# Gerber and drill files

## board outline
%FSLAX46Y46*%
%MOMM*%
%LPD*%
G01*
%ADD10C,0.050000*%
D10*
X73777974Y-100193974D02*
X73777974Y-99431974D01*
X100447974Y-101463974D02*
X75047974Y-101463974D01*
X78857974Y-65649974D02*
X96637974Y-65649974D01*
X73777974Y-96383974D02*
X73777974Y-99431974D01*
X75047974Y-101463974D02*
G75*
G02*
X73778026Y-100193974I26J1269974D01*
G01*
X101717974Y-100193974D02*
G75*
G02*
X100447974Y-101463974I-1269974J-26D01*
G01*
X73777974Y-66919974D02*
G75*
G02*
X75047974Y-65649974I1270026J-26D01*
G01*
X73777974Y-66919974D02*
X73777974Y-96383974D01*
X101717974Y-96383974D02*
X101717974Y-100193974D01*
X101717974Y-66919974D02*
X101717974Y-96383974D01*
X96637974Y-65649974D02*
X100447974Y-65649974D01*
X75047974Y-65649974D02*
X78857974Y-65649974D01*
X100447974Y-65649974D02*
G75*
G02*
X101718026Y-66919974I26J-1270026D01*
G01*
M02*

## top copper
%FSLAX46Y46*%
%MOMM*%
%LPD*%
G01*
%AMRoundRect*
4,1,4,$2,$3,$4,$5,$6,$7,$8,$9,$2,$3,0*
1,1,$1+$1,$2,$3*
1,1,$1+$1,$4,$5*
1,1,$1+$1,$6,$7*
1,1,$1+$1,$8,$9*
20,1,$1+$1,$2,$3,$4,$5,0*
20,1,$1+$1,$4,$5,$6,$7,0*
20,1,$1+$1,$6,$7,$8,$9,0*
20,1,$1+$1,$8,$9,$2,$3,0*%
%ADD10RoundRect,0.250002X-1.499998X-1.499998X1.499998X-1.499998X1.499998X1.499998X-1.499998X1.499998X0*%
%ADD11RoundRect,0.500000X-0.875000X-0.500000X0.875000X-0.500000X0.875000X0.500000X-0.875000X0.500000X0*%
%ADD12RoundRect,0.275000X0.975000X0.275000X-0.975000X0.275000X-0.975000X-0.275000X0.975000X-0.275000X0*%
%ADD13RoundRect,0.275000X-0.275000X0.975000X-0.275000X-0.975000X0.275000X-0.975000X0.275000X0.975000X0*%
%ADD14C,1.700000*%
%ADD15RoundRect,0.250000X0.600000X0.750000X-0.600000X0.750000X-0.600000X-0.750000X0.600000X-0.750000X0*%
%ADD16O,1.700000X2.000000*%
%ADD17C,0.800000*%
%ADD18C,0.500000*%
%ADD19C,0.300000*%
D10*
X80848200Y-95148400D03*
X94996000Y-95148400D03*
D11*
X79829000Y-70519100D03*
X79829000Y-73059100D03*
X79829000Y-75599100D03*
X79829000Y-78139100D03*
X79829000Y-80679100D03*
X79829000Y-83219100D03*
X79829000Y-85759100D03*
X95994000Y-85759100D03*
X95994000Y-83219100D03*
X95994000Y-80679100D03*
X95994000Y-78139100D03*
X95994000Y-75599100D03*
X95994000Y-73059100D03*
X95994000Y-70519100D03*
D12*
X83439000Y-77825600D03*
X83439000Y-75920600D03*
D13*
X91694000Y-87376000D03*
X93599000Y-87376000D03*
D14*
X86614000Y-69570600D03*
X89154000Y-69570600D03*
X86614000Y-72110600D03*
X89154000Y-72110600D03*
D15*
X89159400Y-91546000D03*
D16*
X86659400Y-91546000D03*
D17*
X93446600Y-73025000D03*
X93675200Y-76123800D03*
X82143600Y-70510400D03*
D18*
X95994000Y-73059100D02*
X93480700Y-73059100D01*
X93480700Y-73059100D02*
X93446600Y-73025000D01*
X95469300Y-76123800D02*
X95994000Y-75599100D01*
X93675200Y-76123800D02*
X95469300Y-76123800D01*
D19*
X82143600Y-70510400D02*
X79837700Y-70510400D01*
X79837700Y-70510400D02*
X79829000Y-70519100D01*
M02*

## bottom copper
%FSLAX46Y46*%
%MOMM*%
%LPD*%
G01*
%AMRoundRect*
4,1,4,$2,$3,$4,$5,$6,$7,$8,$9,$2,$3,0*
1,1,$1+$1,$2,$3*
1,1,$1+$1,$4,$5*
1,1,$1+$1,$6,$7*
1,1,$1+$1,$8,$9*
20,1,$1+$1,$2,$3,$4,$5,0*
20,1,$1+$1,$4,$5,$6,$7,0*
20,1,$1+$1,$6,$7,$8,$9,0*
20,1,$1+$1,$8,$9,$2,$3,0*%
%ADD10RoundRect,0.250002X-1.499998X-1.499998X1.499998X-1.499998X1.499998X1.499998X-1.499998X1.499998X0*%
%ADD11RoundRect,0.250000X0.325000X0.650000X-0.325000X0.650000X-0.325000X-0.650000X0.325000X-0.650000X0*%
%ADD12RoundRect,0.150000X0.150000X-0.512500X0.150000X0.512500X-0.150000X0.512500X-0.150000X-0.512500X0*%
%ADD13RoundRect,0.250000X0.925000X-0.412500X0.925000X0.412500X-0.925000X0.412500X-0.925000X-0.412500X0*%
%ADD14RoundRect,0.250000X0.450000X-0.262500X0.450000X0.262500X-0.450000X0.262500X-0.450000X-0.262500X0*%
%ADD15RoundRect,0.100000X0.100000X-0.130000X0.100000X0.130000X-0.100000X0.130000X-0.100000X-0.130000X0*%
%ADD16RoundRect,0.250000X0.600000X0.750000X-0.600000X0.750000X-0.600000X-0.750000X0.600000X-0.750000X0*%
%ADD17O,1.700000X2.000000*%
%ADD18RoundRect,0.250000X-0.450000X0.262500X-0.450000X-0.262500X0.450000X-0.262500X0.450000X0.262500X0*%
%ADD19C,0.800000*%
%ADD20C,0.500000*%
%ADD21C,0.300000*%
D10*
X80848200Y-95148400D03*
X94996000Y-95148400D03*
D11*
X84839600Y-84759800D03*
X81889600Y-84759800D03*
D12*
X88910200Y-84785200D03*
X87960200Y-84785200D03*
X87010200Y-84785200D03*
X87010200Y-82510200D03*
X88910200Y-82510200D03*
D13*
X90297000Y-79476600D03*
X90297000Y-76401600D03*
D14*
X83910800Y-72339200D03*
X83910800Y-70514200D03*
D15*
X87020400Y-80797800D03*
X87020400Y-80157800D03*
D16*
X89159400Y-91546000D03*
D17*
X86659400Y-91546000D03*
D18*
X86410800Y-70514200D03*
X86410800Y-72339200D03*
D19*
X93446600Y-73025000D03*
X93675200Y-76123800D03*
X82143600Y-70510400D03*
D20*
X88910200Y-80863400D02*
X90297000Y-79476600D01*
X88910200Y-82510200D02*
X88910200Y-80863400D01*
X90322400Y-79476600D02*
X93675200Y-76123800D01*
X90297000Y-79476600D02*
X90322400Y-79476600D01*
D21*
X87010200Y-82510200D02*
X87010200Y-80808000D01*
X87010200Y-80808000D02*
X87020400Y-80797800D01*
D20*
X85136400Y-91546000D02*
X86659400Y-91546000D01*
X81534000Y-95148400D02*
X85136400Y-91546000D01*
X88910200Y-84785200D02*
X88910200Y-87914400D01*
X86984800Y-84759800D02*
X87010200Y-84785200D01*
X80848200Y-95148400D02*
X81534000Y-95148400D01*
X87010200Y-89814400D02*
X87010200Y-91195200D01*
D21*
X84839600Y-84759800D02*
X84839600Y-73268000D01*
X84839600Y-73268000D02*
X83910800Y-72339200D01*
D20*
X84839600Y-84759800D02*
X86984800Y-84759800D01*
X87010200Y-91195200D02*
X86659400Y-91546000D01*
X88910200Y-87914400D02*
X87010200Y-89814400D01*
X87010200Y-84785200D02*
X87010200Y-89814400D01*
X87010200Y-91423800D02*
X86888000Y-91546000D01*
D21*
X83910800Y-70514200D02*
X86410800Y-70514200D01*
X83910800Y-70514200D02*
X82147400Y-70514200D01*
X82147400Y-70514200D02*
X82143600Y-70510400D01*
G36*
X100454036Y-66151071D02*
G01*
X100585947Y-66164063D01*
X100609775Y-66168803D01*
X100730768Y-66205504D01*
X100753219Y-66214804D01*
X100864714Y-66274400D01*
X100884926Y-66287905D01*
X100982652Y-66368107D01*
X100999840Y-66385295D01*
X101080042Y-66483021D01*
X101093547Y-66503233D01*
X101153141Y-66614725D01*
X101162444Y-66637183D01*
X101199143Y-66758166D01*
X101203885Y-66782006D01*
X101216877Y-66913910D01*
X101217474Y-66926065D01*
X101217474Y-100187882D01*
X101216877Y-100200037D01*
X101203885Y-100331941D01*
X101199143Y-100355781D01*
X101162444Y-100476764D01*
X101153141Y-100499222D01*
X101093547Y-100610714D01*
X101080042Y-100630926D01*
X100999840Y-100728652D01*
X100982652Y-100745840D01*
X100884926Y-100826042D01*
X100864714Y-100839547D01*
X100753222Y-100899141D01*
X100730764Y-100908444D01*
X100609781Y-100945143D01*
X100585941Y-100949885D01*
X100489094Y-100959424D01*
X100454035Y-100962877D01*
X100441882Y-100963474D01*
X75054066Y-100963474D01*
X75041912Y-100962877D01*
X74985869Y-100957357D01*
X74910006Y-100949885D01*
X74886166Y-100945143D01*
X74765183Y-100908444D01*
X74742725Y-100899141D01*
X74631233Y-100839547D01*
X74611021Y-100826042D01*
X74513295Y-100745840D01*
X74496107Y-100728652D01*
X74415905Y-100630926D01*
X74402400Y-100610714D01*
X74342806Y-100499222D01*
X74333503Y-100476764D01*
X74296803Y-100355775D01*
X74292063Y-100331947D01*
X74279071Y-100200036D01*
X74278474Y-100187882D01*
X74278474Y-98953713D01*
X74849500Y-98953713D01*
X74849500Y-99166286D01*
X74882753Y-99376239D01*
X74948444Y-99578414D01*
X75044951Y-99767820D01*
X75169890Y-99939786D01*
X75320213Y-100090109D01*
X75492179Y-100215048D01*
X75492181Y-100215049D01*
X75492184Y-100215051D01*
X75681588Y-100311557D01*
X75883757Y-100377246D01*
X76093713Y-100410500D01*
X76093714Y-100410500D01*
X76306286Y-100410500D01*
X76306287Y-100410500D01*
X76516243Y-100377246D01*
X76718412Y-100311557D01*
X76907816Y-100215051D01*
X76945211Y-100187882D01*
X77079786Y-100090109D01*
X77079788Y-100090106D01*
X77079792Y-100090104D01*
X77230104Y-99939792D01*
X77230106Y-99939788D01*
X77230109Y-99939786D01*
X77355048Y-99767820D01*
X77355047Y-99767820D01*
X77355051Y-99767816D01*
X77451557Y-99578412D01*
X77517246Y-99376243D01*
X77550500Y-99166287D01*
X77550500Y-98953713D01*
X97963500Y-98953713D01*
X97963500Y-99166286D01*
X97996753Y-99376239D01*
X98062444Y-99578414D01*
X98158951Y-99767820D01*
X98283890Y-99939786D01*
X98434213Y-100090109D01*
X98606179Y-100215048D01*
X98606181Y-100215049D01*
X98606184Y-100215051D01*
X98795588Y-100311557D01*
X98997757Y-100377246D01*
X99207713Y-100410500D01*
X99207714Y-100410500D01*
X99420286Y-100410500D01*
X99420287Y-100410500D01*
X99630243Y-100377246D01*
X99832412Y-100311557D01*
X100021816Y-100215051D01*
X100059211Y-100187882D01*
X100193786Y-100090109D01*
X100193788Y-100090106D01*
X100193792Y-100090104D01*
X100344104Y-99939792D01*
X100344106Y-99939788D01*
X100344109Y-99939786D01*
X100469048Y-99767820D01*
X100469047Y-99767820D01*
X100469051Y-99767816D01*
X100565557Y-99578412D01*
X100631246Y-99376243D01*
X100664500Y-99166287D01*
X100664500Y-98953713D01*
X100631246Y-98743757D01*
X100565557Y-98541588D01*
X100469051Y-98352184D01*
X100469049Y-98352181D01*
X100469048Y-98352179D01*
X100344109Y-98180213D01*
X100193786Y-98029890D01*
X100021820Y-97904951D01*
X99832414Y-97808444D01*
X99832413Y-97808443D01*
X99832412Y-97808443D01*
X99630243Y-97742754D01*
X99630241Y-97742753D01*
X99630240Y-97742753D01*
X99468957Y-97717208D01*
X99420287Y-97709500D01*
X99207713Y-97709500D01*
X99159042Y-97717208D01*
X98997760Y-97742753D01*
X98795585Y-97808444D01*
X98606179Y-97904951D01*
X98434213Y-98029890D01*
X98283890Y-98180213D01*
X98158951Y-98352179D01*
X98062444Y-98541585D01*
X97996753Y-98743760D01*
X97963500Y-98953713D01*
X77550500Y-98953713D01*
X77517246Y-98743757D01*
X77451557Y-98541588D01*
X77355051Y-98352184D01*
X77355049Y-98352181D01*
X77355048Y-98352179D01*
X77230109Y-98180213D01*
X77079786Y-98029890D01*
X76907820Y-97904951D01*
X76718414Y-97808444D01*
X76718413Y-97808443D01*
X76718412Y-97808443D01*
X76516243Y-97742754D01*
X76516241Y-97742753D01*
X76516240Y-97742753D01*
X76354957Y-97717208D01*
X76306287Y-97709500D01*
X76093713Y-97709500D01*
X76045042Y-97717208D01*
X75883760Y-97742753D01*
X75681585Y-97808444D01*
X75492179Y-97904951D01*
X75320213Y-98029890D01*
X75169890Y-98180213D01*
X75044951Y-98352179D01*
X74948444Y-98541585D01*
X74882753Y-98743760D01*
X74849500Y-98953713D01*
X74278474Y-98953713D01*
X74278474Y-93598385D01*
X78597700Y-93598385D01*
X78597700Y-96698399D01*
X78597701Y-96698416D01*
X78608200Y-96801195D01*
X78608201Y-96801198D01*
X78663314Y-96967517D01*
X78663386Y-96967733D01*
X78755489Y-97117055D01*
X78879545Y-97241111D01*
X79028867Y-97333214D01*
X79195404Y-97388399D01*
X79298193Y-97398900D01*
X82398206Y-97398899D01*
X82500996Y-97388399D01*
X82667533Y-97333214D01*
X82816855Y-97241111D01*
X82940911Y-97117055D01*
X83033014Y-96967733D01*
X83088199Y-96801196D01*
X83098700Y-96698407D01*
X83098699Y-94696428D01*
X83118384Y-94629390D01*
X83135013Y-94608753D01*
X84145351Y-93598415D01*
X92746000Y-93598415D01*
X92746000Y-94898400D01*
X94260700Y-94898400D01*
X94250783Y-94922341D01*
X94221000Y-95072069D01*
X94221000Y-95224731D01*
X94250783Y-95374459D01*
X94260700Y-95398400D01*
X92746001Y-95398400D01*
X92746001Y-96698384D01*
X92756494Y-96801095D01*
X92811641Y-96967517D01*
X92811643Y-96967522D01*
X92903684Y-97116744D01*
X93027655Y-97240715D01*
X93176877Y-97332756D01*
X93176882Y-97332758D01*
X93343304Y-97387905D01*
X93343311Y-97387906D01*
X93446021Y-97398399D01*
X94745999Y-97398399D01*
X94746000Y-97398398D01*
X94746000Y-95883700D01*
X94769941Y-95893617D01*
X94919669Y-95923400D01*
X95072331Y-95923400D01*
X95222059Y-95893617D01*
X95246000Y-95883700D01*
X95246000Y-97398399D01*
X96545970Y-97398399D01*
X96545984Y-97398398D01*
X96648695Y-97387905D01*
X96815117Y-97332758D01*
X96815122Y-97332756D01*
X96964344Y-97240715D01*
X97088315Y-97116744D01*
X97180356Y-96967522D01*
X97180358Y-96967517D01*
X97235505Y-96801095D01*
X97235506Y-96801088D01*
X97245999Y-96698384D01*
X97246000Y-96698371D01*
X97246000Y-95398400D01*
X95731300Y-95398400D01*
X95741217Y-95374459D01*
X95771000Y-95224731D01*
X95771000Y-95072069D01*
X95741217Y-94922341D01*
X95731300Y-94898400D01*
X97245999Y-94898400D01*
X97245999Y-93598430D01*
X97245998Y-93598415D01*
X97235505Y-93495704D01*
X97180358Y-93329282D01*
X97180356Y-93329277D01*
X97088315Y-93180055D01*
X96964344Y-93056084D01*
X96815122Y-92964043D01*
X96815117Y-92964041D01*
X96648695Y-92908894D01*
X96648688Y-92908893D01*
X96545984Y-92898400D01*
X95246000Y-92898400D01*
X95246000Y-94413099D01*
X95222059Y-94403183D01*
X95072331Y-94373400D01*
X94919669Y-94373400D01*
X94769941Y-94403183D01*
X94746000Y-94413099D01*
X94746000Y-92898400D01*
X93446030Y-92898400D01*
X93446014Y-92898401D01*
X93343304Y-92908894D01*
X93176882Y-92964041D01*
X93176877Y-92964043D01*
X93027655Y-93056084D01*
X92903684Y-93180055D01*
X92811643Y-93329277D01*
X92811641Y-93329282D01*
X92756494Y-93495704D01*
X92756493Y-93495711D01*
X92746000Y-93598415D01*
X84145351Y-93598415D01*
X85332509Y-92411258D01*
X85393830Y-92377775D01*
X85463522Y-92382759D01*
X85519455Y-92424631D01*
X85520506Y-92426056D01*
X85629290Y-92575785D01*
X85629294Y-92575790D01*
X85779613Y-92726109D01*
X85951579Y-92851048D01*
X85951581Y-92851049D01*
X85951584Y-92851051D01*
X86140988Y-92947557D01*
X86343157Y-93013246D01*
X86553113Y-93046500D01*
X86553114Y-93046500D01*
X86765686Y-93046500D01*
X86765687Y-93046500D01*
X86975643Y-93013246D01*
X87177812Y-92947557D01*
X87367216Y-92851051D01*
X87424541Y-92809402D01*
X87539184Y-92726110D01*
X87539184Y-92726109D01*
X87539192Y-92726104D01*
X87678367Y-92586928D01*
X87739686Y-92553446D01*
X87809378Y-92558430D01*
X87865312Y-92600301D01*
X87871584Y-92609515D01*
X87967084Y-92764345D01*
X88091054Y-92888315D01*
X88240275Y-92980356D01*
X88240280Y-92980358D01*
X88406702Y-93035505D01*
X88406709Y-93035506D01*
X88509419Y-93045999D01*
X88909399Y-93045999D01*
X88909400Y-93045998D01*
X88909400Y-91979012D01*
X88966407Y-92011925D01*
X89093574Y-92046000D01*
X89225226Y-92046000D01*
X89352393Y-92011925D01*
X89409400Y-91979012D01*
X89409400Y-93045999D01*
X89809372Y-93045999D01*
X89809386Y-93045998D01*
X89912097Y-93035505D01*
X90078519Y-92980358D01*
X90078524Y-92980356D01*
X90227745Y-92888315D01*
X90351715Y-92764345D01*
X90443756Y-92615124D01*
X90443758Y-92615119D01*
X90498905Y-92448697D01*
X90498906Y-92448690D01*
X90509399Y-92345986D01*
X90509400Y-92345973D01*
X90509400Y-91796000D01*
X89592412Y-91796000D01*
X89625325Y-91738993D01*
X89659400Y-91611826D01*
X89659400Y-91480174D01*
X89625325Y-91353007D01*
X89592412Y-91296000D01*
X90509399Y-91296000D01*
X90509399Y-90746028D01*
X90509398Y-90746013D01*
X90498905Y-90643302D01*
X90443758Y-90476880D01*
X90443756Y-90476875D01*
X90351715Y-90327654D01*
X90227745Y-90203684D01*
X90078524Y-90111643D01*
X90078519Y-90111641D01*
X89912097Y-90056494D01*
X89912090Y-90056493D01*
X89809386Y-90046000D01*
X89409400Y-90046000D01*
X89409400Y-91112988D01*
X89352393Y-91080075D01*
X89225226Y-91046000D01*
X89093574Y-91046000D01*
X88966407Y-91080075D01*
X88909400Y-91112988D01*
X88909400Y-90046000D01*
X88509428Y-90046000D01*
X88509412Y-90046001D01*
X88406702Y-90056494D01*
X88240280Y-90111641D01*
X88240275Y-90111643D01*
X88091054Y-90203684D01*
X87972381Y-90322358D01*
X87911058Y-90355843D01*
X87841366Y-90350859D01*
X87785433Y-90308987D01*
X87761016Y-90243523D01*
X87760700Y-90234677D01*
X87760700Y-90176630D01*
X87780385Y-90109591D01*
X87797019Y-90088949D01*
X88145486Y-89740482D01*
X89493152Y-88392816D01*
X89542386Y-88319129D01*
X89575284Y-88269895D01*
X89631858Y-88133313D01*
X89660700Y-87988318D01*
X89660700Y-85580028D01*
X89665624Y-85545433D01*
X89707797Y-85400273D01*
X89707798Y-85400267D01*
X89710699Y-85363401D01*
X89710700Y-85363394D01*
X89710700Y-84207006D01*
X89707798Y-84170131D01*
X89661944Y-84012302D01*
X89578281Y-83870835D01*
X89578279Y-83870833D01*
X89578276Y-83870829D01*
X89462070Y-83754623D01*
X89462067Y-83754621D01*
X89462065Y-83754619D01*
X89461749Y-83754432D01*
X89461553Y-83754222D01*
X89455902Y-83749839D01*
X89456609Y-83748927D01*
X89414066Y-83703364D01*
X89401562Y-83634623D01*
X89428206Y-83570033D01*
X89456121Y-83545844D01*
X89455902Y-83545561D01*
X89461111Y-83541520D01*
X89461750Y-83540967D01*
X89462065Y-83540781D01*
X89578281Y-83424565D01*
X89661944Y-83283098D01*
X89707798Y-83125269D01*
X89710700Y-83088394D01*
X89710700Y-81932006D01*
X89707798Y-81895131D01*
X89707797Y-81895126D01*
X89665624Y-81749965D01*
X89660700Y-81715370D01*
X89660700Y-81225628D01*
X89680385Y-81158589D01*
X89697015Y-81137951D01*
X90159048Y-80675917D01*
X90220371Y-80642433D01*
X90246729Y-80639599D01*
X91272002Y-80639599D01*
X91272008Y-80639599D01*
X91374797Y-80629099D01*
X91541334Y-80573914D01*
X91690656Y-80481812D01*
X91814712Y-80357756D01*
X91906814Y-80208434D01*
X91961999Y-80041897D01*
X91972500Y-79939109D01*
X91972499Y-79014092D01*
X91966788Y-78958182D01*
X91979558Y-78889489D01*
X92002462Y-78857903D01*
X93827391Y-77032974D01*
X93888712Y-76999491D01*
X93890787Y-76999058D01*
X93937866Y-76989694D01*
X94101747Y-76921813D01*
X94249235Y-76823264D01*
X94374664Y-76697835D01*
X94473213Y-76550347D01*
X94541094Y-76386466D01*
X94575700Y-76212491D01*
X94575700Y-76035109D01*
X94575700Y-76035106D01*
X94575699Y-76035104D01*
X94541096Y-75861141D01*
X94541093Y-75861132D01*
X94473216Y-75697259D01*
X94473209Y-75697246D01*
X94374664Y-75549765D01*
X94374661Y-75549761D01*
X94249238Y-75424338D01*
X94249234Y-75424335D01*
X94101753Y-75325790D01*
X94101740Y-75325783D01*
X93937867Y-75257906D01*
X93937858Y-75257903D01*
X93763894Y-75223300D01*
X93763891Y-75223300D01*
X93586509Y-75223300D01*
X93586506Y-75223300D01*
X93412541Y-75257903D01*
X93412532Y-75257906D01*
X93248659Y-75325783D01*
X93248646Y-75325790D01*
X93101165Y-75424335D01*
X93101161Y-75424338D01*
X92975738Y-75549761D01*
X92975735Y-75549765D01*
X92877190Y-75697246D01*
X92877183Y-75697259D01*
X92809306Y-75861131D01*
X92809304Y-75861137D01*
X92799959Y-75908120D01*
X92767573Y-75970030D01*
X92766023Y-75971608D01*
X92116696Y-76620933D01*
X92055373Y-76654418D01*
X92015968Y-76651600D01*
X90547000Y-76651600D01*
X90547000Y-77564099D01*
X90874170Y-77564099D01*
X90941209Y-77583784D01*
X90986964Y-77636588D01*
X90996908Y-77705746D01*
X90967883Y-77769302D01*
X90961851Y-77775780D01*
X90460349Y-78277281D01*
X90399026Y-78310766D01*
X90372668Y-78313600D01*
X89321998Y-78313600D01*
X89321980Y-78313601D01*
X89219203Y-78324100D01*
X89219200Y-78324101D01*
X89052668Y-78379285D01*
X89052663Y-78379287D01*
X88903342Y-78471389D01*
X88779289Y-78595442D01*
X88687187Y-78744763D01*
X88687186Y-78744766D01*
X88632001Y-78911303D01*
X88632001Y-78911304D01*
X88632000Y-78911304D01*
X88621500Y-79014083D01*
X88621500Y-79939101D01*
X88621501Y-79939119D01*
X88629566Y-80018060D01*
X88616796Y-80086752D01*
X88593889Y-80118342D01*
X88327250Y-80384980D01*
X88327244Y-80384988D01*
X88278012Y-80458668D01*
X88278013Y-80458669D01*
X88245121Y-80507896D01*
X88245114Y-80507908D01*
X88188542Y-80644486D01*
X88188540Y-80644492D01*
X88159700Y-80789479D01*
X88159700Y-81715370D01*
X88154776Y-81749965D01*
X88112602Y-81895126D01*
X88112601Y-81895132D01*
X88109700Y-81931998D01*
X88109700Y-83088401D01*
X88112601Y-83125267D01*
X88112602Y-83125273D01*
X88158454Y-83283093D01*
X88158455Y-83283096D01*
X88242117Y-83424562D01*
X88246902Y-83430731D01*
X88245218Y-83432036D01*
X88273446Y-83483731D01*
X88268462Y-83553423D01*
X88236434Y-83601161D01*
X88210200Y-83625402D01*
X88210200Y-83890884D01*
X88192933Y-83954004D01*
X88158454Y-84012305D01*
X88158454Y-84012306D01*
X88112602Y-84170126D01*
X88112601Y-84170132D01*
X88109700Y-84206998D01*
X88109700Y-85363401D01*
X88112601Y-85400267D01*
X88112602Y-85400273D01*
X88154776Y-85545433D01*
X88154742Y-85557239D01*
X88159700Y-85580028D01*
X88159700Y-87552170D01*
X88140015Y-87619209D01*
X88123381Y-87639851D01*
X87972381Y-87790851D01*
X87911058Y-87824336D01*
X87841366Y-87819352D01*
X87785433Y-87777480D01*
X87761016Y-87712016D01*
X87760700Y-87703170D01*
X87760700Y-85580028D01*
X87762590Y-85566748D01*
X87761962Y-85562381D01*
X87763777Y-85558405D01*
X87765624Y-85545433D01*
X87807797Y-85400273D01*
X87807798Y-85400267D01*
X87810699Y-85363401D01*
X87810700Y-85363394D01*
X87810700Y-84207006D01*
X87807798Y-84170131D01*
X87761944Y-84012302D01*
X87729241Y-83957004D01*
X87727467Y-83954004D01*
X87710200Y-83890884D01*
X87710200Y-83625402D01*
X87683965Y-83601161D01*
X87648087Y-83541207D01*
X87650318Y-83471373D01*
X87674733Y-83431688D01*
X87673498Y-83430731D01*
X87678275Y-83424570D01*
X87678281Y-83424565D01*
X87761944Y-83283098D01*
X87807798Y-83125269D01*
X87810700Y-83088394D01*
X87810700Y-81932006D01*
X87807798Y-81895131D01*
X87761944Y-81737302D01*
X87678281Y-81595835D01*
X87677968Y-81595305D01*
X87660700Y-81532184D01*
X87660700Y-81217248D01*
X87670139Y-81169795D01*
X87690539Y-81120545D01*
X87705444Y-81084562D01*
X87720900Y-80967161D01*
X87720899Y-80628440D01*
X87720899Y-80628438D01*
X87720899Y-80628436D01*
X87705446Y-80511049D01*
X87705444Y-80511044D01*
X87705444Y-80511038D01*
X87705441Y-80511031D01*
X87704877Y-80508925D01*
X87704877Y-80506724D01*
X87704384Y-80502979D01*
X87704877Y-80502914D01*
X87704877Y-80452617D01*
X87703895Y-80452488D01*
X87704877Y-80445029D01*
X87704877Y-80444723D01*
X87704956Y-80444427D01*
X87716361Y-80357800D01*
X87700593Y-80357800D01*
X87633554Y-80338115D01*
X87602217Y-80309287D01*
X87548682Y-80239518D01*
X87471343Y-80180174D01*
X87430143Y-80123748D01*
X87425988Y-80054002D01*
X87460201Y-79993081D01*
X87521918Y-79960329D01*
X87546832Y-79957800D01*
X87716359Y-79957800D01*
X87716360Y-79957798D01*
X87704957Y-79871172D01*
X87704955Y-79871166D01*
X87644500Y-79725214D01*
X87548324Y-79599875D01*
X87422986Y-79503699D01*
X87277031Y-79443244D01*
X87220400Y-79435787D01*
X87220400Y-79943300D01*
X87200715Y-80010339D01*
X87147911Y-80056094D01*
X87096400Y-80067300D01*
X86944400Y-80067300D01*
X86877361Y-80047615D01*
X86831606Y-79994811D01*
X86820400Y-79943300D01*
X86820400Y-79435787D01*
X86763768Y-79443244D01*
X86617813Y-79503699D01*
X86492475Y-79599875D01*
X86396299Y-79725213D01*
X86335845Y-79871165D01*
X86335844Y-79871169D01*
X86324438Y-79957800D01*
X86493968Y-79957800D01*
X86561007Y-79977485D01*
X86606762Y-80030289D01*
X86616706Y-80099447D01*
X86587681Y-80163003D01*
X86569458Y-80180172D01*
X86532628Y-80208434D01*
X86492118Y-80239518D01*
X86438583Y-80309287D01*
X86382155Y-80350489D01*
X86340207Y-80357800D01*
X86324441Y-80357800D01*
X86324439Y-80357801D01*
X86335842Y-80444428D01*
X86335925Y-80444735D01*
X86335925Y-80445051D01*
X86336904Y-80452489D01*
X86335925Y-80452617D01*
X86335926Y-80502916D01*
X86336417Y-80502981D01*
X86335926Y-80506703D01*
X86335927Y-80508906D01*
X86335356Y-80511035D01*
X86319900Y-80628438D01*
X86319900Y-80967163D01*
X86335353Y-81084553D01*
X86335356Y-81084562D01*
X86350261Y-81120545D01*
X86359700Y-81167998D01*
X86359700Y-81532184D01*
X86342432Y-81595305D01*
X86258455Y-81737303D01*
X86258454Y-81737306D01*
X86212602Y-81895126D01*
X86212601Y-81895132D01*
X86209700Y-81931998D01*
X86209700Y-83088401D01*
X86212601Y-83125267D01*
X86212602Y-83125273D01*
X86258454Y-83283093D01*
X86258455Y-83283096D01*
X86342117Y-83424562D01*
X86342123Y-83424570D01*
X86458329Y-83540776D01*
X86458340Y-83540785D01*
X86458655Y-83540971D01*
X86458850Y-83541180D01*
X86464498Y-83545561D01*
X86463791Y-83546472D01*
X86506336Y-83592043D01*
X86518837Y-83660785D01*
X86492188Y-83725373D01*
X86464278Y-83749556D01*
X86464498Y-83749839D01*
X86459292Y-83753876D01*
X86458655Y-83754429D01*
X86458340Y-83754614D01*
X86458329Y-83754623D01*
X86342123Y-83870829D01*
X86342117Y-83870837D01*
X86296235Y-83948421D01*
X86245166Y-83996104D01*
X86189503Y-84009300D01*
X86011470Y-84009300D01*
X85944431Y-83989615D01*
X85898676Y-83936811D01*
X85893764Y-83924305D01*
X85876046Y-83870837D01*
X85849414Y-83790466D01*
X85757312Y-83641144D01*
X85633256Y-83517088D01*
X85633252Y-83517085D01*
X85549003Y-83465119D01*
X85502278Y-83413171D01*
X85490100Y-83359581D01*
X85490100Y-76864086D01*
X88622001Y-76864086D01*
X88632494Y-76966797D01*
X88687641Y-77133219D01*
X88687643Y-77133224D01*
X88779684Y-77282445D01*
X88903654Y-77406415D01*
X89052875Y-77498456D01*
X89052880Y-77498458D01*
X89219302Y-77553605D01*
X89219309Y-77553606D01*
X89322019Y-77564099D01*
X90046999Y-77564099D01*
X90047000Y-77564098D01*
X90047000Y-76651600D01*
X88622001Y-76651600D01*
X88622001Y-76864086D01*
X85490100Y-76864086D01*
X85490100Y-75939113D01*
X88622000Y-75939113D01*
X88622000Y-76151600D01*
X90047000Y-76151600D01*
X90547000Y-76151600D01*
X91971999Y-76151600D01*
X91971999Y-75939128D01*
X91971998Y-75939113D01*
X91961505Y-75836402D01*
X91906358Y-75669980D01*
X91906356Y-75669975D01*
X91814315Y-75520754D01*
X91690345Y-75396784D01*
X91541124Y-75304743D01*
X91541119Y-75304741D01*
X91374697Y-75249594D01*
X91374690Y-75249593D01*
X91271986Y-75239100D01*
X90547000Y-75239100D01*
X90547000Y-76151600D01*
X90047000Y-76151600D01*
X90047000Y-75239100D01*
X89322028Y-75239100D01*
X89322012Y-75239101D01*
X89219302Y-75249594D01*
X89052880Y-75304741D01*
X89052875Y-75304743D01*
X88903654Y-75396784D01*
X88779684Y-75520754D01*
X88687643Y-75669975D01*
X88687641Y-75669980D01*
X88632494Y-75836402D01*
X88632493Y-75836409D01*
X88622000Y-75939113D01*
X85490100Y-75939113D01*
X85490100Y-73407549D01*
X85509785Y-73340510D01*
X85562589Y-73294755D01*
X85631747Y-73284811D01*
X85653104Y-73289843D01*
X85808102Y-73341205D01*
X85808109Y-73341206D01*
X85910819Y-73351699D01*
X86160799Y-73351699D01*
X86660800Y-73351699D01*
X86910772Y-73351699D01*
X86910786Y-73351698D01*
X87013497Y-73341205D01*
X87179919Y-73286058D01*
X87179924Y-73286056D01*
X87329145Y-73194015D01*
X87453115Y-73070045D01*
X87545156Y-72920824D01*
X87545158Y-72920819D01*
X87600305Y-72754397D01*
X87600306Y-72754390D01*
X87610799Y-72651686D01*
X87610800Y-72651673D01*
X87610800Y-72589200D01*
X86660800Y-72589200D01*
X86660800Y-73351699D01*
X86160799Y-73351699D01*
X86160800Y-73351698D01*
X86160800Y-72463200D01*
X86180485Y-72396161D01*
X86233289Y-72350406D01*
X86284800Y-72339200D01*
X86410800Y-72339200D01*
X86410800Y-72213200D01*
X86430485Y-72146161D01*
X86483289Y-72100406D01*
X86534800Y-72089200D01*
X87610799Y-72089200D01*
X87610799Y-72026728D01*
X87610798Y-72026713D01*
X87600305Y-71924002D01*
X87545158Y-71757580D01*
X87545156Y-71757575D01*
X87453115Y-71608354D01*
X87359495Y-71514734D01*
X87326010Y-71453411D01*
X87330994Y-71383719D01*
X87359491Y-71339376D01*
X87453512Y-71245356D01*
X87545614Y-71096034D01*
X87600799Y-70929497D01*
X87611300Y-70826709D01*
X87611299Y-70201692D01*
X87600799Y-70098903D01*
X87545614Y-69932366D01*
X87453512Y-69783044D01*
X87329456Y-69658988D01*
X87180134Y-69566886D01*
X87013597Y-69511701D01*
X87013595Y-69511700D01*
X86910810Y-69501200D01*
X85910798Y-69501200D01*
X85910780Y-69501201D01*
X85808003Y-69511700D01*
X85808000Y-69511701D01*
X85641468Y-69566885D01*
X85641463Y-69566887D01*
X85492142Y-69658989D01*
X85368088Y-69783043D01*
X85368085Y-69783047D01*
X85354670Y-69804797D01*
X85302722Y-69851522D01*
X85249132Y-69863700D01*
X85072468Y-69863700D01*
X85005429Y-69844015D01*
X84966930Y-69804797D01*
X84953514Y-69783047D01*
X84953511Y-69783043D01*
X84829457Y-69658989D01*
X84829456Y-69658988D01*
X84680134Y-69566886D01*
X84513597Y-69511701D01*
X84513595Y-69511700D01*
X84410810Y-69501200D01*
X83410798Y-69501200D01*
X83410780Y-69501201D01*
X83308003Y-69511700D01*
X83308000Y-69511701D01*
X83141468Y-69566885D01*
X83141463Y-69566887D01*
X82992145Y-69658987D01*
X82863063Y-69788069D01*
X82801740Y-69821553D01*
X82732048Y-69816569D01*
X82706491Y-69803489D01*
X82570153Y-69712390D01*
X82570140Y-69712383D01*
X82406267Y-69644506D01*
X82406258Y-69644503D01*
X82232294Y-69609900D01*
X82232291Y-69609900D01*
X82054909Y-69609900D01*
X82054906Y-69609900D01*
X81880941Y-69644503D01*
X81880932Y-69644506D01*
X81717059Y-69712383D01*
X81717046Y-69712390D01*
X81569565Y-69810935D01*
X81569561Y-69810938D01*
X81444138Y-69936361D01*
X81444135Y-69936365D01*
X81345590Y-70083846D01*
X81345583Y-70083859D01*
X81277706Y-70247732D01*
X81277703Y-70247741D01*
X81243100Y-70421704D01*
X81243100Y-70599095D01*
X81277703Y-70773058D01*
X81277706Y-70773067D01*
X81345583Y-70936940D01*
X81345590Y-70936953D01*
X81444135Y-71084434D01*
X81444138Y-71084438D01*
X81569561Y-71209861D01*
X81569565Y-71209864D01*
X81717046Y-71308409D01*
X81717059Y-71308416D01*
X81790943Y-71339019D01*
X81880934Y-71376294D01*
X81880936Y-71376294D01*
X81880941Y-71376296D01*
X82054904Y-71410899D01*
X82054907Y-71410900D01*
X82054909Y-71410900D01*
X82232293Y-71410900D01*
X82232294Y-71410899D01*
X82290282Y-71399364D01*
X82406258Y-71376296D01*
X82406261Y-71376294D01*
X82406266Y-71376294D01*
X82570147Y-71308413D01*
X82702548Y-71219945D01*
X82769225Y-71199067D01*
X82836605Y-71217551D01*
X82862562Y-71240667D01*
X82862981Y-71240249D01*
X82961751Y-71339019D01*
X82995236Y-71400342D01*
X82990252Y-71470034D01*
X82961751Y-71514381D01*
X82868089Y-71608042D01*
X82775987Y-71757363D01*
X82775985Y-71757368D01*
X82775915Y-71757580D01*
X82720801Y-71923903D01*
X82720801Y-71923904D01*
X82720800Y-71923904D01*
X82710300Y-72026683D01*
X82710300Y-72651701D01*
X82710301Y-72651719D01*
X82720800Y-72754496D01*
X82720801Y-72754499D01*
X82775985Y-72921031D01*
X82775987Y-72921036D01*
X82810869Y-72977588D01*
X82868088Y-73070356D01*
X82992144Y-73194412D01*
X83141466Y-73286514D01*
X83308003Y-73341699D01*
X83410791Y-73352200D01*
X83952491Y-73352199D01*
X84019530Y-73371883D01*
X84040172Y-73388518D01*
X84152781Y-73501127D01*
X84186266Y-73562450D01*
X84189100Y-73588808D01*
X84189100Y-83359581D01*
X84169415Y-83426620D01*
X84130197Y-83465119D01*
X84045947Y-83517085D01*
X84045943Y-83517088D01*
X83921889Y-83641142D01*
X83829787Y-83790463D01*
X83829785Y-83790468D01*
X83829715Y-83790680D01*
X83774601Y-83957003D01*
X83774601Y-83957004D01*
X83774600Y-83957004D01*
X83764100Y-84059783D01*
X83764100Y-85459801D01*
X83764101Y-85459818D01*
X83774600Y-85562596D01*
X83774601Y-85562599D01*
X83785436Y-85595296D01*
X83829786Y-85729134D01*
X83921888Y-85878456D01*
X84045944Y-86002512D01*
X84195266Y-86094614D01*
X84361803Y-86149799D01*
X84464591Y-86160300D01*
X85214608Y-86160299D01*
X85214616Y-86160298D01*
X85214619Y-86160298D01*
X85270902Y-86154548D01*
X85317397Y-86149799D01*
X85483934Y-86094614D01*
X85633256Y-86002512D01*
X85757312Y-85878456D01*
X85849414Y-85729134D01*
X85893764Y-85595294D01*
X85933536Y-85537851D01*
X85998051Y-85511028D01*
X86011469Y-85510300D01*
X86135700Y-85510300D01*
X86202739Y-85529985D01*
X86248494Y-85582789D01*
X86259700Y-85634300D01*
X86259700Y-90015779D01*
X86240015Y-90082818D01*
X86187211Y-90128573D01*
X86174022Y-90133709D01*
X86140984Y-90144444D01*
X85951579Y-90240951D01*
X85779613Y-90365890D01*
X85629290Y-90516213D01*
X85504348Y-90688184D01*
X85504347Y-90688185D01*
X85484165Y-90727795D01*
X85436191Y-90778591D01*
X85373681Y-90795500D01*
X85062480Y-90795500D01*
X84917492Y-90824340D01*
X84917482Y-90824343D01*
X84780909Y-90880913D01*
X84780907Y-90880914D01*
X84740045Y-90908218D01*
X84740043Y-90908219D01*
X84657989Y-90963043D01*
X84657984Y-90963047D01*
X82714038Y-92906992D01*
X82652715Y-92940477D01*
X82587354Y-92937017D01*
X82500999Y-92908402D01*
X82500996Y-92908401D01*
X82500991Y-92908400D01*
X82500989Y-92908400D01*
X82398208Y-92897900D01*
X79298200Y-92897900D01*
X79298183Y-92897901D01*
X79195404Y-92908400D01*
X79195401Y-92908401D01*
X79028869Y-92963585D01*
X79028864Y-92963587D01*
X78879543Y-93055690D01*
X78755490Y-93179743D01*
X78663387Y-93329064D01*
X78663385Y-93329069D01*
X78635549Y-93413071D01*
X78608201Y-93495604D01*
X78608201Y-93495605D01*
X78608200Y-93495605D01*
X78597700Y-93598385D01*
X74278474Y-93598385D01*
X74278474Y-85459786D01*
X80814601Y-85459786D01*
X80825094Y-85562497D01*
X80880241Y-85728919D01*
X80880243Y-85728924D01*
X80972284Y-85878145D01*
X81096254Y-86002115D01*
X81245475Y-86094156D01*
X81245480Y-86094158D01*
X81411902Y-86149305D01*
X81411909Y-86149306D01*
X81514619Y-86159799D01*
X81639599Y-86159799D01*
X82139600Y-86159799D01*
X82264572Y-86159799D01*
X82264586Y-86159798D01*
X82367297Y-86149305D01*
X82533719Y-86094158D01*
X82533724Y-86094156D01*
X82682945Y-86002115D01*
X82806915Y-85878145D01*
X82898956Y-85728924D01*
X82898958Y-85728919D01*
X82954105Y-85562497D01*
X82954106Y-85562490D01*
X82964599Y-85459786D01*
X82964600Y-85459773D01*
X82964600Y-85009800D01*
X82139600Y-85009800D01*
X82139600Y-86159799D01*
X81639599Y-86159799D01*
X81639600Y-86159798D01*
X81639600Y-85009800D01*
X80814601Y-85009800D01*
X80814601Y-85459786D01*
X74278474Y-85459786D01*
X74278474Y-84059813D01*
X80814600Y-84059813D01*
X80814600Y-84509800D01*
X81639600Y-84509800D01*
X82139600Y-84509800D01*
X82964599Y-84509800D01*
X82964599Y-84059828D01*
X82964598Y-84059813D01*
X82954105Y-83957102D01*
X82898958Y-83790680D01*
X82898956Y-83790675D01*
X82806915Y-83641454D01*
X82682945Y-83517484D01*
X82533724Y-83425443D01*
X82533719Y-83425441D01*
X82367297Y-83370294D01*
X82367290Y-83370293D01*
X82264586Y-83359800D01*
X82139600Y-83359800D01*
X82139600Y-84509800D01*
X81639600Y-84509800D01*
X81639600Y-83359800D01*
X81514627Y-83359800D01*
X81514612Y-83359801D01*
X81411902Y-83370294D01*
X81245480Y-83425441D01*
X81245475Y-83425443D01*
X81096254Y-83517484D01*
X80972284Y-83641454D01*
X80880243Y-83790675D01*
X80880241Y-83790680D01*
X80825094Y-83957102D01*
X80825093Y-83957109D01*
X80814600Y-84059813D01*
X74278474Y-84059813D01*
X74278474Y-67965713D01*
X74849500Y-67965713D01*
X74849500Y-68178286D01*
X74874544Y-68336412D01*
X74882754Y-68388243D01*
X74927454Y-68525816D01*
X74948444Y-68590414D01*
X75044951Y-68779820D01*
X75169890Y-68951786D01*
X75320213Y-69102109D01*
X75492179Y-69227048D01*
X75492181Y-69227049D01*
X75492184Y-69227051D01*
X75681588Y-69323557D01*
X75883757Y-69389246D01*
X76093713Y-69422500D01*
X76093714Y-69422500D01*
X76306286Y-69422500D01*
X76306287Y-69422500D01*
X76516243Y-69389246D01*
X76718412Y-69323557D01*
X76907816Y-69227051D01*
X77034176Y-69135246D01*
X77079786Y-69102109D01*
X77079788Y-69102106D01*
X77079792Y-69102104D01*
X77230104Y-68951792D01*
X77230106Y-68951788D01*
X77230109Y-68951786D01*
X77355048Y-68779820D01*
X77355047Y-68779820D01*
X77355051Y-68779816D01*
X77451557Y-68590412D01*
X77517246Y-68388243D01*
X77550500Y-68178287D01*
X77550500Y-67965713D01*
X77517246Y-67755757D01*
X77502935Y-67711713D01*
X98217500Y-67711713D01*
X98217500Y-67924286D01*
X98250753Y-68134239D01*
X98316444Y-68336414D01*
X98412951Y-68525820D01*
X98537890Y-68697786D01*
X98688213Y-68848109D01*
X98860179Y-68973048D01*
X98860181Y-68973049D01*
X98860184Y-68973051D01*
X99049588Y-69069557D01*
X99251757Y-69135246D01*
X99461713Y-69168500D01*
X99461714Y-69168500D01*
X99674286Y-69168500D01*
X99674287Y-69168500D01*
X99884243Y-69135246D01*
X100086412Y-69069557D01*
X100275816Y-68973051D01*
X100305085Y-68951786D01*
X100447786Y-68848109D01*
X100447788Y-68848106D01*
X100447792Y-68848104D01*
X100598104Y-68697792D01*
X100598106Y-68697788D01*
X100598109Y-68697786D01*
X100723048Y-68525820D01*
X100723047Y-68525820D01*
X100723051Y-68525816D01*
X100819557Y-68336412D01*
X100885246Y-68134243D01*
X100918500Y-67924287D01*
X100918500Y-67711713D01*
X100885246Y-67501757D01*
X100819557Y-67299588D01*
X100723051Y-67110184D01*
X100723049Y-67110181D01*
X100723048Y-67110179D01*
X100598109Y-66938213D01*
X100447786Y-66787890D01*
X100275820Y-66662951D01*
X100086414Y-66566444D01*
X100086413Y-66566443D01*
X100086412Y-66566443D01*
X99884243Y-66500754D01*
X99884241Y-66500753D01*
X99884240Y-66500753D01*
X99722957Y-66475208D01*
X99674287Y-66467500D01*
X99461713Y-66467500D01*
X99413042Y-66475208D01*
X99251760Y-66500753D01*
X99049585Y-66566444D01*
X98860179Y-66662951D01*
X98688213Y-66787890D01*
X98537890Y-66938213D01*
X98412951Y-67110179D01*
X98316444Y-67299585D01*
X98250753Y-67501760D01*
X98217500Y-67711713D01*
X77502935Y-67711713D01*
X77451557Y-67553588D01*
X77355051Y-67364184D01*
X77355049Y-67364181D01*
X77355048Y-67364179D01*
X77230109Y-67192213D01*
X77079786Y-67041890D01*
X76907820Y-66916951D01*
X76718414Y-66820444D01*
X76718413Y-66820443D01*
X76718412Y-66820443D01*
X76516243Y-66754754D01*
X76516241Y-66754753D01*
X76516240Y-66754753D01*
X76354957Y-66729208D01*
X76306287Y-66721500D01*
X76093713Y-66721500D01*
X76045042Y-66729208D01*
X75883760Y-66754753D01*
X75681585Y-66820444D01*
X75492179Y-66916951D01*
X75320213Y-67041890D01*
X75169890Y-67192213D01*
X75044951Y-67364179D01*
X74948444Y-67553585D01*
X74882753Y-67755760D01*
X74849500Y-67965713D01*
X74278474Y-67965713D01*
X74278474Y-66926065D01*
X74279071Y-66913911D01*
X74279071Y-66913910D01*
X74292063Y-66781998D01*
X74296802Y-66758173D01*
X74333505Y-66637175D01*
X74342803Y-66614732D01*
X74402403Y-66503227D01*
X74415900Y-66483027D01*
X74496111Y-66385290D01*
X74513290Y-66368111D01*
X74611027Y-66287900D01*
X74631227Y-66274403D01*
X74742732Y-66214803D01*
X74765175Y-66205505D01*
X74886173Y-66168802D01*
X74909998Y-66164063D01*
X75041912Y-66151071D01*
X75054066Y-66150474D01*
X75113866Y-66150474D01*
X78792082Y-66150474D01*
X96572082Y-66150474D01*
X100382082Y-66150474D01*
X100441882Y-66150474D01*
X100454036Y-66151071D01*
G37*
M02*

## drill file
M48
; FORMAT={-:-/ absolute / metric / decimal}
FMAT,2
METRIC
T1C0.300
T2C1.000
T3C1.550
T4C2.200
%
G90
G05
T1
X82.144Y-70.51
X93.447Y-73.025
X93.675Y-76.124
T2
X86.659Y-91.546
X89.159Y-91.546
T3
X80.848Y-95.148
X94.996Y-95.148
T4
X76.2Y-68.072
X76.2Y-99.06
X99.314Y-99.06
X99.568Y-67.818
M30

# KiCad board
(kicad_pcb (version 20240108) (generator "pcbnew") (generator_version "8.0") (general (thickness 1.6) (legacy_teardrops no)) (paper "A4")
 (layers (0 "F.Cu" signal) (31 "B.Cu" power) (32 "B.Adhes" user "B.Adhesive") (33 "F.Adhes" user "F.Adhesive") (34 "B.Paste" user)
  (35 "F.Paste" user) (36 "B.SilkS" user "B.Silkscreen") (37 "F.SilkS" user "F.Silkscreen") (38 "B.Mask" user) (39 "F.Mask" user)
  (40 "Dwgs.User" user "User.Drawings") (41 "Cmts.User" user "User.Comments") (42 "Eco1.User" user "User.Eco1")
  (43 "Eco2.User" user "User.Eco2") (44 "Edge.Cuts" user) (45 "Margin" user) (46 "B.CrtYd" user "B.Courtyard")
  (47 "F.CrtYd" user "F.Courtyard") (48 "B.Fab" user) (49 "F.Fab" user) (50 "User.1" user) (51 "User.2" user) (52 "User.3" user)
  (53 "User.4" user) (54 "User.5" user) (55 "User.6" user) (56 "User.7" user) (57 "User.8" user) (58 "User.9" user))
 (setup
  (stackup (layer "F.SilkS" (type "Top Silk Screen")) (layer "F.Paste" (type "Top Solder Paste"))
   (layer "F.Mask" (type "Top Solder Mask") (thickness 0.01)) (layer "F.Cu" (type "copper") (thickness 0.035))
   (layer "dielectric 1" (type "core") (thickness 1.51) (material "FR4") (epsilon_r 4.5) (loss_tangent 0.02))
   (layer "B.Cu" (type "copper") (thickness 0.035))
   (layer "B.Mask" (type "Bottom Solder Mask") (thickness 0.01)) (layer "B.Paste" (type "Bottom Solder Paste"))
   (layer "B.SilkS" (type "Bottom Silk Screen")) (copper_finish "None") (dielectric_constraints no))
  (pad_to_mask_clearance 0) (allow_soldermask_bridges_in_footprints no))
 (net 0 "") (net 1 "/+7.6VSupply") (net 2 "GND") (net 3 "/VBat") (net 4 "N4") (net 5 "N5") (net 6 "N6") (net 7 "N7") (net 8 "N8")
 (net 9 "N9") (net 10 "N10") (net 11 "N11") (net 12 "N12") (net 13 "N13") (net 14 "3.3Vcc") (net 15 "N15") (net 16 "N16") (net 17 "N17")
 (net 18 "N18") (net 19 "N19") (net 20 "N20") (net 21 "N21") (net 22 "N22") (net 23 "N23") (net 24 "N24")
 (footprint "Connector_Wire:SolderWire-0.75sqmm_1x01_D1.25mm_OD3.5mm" (layer "F.Cu") (at 80.8482 95.1484)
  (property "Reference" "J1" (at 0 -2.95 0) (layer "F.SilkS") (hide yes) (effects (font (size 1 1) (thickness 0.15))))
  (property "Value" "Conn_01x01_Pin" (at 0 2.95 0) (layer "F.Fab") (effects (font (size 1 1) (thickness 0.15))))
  (pad "1" thru_hole roundrect (at 0 0) (size 3.5 3.5) (drill 1.55) (layers "*.Cu" "*.Mask") (remove_unused_layers no)
   (roundrect_rratio 0.071429) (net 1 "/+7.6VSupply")))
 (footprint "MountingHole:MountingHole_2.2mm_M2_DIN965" (layer "F.Cu") (at 99.568 67.818)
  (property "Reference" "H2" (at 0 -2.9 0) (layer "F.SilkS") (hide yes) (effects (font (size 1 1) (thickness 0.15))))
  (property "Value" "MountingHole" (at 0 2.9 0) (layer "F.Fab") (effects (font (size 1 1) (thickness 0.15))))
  (pad "" np_thru_hole circle (at 0 0) (size 2.2 2.2) (drill 2.2) (layers "*.Cu" "*.Mask")))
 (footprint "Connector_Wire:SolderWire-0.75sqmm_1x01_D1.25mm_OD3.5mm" (layer "F.Cu") (at 94.996 95.1484)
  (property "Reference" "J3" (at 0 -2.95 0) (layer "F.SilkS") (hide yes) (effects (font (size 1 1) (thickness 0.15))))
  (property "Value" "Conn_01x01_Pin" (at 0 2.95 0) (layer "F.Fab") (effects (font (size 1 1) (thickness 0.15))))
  (pad "1" thru_hole roundrect (at 0 0) (size 3.5 3.5) (drill 1.55) (layers "*.Cu" "*.Mask") (remove_unused_layers no)
   (roundrect_rratio 0.071429) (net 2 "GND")))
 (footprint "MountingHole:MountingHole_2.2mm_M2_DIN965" (layer "F.Cu") (at 76.2 99.06)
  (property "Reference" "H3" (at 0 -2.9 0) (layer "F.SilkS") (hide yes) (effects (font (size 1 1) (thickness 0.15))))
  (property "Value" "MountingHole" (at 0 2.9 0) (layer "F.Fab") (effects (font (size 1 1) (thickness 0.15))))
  (pad "" np_thru_hole circle (at 0 0) (size 2.2 2.2) (drill 2.2) (layers "*.Cu" "*.Mask")))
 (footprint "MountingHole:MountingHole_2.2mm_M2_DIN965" (layer "F.Cu") (at 99.314 99.06)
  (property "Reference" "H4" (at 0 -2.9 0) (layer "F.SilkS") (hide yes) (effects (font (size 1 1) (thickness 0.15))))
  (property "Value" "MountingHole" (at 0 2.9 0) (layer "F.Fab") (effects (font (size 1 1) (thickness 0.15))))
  (pad "" np_thru_hole circle (at 0 0) (size 2.2 2.2) (drill 2.2) (layers "*.Cu" "*.Mask")))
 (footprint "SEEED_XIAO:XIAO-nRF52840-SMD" (layer "F.Cu") (at 78.994 88.6391)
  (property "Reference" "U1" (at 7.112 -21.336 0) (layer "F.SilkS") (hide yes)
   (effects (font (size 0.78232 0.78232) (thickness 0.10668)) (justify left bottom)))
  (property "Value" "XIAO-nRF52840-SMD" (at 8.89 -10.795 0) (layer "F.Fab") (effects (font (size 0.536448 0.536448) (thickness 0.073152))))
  (pad "1" smd roundrect (at 0.835 -18.12) (size 2.75 2) (layers "F.Cu" "F.Paste" "F.Mask") (roundrect_rratio 0.25) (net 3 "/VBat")
   (solder_mask_margin 0.0508) (thermal_bridge_angle 45))
  (pad "2" smd roundrect (at 0.835 -15.58) (size 2.75 2) (layers "F.Cu" "F.Paste" "F.Mask") (roundrect_rratio 0.25) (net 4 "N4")
   (solder_mask_margin 0.0508) (thermal_bridge_angle 45))
  (pad "3" smd roundrect (at 0.835 -13.04) (size 2.75 2) (layers "F.Cu" "F.Paste" "F.Mask") (roundrect_rratio 0.25) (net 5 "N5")
   (solder_mask_margin 0.0508) (thermal_bridge_angle 45))
  (pad "4" smd roundrect (at 0.835 -10.5) (size 2.75 2) (layers "F.Cu" "F.Paste" "F.Mask") (roundrect_rratio 0.25) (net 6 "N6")
   (solder_mask_margin 0.0508) (thermal_bridge_angle 45))
  (pad "5" smd roundrect (at 0.835 -7.96) (size 2.75 2) (layers "F.Cu" "F.Paste" "F.Mask") (roundrect_rratio 0.25) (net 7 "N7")
   (solder_mask_margin 0.0508) (thermal_bridge_angle 45))
  (pad "6" smd roundrect (at 0.835 -5.42) (size 2.75 2) (layers "F.Cu" "F.Paste" "F.Mask") (roundrect_rratio 0.25) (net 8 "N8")
   (solder_mask_margin 0.0508) (thermal_bridge_angle 45))
  (pad "7" smd roundrect (at 0.835 -2.88) (size 2.75 2) (layers "F.Cu" "F.Paste" "F.Mask") (roundrect_rratio 0.25) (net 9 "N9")
   (solder_mask_margin 0.0508) (thermal_bridge_angle 45))
  (pad "8" smd roundrect (at 17 -2.88) (size 2.75 2) (layers "F.Cu" "F.Paste" "F.Mask") (roundrect_rratio 0.25) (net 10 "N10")
   (solder_mask_margin 0.0508) (thermal_bridge_angle 45))
  (pad "9" smd roundrect (at 17 -5.42) (size 2.75 2) (layers "F.Cu" "F.Paste" "F.Mask") (roundrect_rratio 0.25) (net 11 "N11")
   (solder_mask_margin 0.0508) (thermal_bridge_angle 45))
  (pad "10" smd roundrect (at 17 -7.96) (size 2.75 2) (layers "F.Cu" "F.Paste" "F.Mask") (roundrect_rratio 0.25) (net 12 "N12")
   (solder_mask_margin 0.0508) (thermal_bridge_angle 45))
  (pad "11" smd roundrect (at 17 -10.5) (size 2.75 2) (layers "F.Cu" "F.Paste" "F.Mask") (roundrect_rratio 0.25) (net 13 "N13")
   (solder_mask_margin 0.0508) (thermal_bridge_angle 45))
  (pad "12" smd roundrect (at 17 -13.04) (size 2.75 2) (layers "F.Cu" "F.Paste" "F.Mask") (roundrect_rratio 0.25) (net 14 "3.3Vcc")
   (solder_mask_margin 0.0508) (thermal_bridge_angle 45))
  (pad "13" smd roundrect (at 17 -15.58) (size 2.75 2) (layers "F.Cu" "F.Paste" "F.Mask") (roundrect_rratio 0.25) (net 2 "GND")
   (solder_mask_margin 0.0508) (thermal_bridge_angle 45))
  (pad "14" smd roundrect (at 17 -18.12) (size 2.75 2) (layers "F.Cu" "F.Paste" "F.Mask") (roundrect_rratio 0.25) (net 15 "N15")
   (solder_mask_margin 0.0508) (thermal_bridge_angle 45))
  (pad "15" smd roundrect (at 4.445 -10.8135 180) (size 2.5 1.1) (layers "F.Cu" "F.Paste" "F.Mask") (roundrect_rratio 0.25) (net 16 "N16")
   (solder_mask_margin 0.0508) (thermal_bridge_angle 45))
  (pad "16" smd roundrect (at 4.445 -12.7185 180) (size 2.5 1.1) (layers "F.Cu" "F.Paste" "F.Mask") (roundrect_rratio 0.25) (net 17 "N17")
   (solder_mask_margin 0.0508) (thermal_bridge_angle 45))
  (pad "17" smd roundrect (at 12.7 -1.2631 270) (size 2.5 1.1) (layers "F.Cu" "F.Paste" "F.Mask") (roundrect_rratio 0.25) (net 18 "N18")
   (solder_mask_margin 0.0508) (thermal_bridge_angle 45))
  (pad "18" smd roundrect (at 14.605 -1.2631 270) (size 2.5 1.1) (layers "F.Cu" "F.Paste" "F.Mask") (roundrect_rratio 0.25) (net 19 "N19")
   (solder_mask_margin 0.0508) (thermal_bridge_angle 45))
  (pad "19" smd circle (at 7.62 -19.0685) (size 1.7 1.7) (layers "F.Cu" "F.Paste" "F.Mask") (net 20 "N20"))
  (pad "20" smd circle (at 10.16 -19.0685) (size 1.7 1.7) (layers "F.Cu" "F.Paste" "F.Mask") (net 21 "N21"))
  (pad "21" smd circle (at 7.62 -16.5285) (size 1.7 1.7) (layers "F.Cu" "F.Paste" "F.Mask") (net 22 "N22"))
  (pad "22" smd circle (at 10.16 -16.5285) (size 1.7 1.7) (layers "F.Cu" "F.Paste" "F.Mask") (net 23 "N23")))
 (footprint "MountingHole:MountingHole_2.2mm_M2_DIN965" (layer "F.Cu") (at 76.2 68.072)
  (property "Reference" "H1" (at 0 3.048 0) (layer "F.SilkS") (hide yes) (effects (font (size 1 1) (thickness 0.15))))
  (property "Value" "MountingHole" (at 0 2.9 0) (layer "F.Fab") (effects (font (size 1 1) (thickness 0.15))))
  (pad "" np_thru_hole circle (at 0 0) (size 2.2 2.2) (drill 2.2) (layers "*.Cu" "*.Mask")))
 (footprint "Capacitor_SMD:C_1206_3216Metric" (layer "B.Cu") (at 83.3646 84.7598 180)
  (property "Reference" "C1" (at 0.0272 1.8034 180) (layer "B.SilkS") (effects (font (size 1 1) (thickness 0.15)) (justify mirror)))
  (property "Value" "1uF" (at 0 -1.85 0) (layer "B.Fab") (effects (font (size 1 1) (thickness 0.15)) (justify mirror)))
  (pad "1" smd roundrect (at -1.475 0 180) (size 1.15 1.8) (layers "B.Cu" "B.Paste" "B.Mask") (roundrect_rratio 0.217391)
   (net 1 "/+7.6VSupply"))
  (pad "2" smd roundrect (at 1.475 0 180) (size 1.15 1.8) (layers "B.Cu" "B.Paste" "B.Mask") (roundrect_rratio 0.217391) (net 2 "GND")))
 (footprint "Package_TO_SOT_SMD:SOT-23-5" (layer "B.Cu") (at 87.9602 83.6477 90)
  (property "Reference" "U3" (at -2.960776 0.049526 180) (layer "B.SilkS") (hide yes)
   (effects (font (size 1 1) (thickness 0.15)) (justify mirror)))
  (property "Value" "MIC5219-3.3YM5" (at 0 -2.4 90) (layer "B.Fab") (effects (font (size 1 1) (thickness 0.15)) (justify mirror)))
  (pad "1" smd roundrect (at -1.1375 0.95 90) (size 1.325 0.6) (layers "B.Cu" "B.Paste" "B.Mask") (roundrect_rratio 0.25)
   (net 1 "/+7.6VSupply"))
  (pad "2" smd roundrect (at -1.1375 0 90) (size 1.325 0.6) (layers "B.Cu" "B.Paste" "B.Mask") (roundrect_rratio 0.25) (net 2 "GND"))
  (pad "3" smd roundrect (at -1.1375 -0.95 90) (size 1.325 0.6) (layers "B.Cu" "B.Paste" "B.Mask") (roundrect_rratio 0.25)
   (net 1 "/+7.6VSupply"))
  (pad "4" smd roundrect (at 1.1375 -0.95 90) (size 1.325 0.6) (layers "B.Cu" "B.Paste" "B.Mask") (roundrect_rratio 0.25) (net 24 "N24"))
  (pad "5" smd roundrect (at 1.1375 0.95 90) (size 1.325 0.6) (layers "B.Cu" "B.Paste" "B.Mask") (roundrect_rratio 0.25) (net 14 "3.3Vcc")))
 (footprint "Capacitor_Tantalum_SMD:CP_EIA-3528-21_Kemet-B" (layer "B.Cu") (at 90.297 77.9391 90)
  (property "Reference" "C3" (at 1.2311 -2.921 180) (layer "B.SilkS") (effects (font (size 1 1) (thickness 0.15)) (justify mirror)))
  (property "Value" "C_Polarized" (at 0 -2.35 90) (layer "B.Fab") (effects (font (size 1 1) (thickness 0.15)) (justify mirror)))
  (pad "1" smd roundrect (at -1.5375 0 90) (size 1.325 2.35) (layers "B.Cu" "B.Paste" "B.Mask") (roundrect_rratio 0.188679)
   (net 14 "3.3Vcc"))
  (pad "2" smd roundrect (at 1.5375 0 90) (size 1.325 2.35) (layers "B.Cu" "B.Paste" "B.Mask") (roundrect_rratio 0.188679) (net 2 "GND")))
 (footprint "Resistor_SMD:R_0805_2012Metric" (layer "B.Cu") (at 83.9108 71.4267 90)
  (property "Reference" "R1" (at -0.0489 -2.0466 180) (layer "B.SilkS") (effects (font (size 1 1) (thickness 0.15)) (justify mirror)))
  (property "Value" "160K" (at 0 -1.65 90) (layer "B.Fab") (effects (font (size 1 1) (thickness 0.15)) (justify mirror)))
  (pad "1" smd roundrect (at -0.9125 0 90) (size 1.025 1.4) (layers "B.Cu" "B.Paste" "B.Mask") (roundrect_rratio 0.243902)
   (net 1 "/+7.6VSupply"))
  (pad "2" smd roundrect (at 0.9125 0 90) (size 1.025 1.4) (layers "B.Cu" "B.Paste" "B.Mask") (roundrect_rratio 0.243902) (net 3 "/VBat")))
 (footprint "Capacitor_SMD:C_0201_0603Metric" (layer "B.Cu") (at 87.0204 80.4778 90)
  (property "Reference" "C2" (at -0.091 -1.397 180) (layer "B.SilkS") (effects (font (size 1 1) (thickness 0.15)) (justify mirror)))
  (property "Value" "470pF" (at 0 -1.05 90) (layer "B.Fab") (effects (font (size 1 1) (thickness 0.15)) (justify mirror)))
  (pad "" smd roundrect (at -0.345 0 90) (size 0.318 0.36) (layers "B.Paste") (roundrect_rratio 0.25))
  (pad "" smd roundrect (at 0.345 0 90) (size 0.318 0.36) (layers "B.Paste") (roundrect_rratio 0.25))
  (pad "1" smd roundrect (at -0.32 0 90) (size 0.46 0.4) (layers "B.Cu" "B.Mask") (roundrect_rratio 0.25) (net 24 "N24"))
  (pad "2" smd roundrect (at 0.32 0 90) (size 0.46 0.4) (layers "B.Cu" "B.Mask") (roundrect_rratio 0.25) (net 2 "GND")))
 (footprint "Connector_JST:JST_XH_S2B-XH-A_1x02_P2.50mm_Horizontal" (layer "B.Cu") (at 89.1594 91.546 180)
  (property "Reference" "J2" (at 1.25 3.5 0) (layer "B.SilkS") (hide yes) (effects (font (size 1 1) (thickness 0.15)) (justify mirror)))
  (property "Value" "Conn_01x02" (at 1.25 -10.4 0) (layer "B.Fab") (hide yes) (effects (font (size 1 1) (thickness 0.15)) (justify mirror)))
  (pad "1" thru_hole roundrect (at 0 0 180) (size 1.7 2) (drill 1) (layers "*.Cu" "*.Mask") (remove_unused_layers no)
   (roundrect_rratio 0.147059) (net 2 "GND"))
  (pad "2" thru_hole oval (at 2.5 0 180) (size 1.7 2) (drill 1) (layers "*.Cu" "*.Mask") (remove_unused_layers no) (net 1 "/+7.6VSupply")))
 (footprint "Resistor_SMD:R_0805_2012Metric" (layer "B.Cu") (at 86.4108 71.4267 -90)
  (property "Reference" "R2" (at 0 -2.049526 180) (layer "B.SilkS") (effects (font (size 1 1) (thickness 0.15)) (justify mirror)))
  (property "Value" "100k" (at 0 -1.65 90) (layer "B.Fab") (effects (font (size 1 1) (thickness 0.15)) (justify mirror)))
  (pad "1" smd roundrect (at -0.9125 0 270) (size 1.025 1.4) (layers "B.Cu" "B.Paste" "B.Mask") (roundrect_rratio 0.243902) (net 3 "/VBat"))
  (pad "2" smd roundrect (at 0.9125 0 270) (size 1.025 1.4) (layers "B.Cu" "B.Paste" "B.Mask") (roundrect_rratio 0.243902) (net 2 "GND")))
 (gr_line (start 73.777974 100.193974) (end 73.777974 99.431974) (stroke (width 0.05) (type default)) (layer "Edge.Cuts"))
 (gr_line (start 100.447974 101.463974) (end 75.047974 101.463974) (stroke (width 0.05) (type default)) (layer "Edge.Cuts"))
 (gr_line (start 78.857974 65.649974) (end 96.637974 65.649974) (stroke (width 0.05) (type default)) (layer "Edge.Cuts"))
 (gr_line (start 73.777974 96.383974) (end 73.777974 99.431974) (stroke (width 0.05) (type default)) (layer "Edge.Cuts"))
 (gr_arc (start 75.047974 101.463974) (mid 74.149948 101.092) (end 73.777974 100.193974) (stroke (width 0.05) (type default))
  (layer "Edge.Cuts"))
 (gr_arc (start 101.717974 100.193974) (mid 101.346 101.092) (end 100.447974 101.463974) (stroke (width 0.05) (type default))
  (layer "Edge.Cuts"))
 (gr_arc (start 73.777974 66.919974) (mid 74.149948 66.021948) (end 75.047974 65.649974) (stroke (width 0.05) (type default))
  (layer "Edge.Cuts"))
 (gr_line (start 73.777974 66.919974) (end 73.777974 96.383974) (stroke (width 0.05) (type default)) (layer "Edge.Cuts"))
 (gr_line (start 101.717974 96.383974) (end 101.717974 100.193974) (stroke (width 0.05) (type default)) (layer "Edge.Cuts"))
 (gr_line (start 101.717974 66.919974) (end 101.717974 96.383974) (stroke (width 0.05) (type default)) (layer "Edge.Cuts"))
 (gr_line (start 96.637974 65.649974) (end 100.447974 65.649974) (stroke (width 0.05) (type default)) (layer "Edge.Cuts"))
 (gr_line (start 75.047974 65.649974) (end 78.857974 65.649974) (stroke (width 0.05) (type default)) (layer "Edge.Cuts"))
 (gr_arc (start 100.447974 65.649974) (mid 101.346 66.021948) (end 101.717974 66.919974) (stroke (width 0.05) (type default))
  (layer "Edge.Cuts"))
 (segment (start 95.994 73.0591) (end 93.4807 73.0591) (width 0.5) (layer "F.Cu") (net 2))
 (segment (start 93.4807 73.0591) (end 93.4466 73.025) (width 0.5) (layer "F.Cu") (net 2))
 (via (at 93.4466 73.025) (size 0.8) (drill 0.3) (layers "F.Cu" "B.Cu") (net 2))
 (segment (start 95.4693 76.1238) (end 95.994 75.5991) (width 0.5) (layer "F.Cu") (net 14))
 (segment (start 93.6752 76.1238) (end 95.4693 76.1238) (width 0.5) (layer "F.Cu") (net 14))
 (via (at 93.6752 76.1238) (size 0.8) (drill 0.3) (layers "F.Cu" "B.Cu") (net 14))
 (segment (start 88.9102 80.8634) (end 90.297 79.4766) (width 0.5) (layer "B.Cu") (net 14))
 (segment (start 88.9102 82.5102) (end 88.9102 80.8634) (width 0.5) (layer "B.Cu") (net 14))
 (segment (start 90.3224 79.4766) (end 93.6752 76.1238) (width 0.5) (layer "B.Cu") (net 14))
 (segment (start 90.297 79.4766) (end 90.3224 79.4766) (width 0.5) (layer "B.Cu") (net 14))
 (segment (start 87.0102 82.5102) (end 87.0102 80.808) (width 0.3) (layer "B.Cu") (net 24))
 (segment (start 87.0102 80.808) (end 87.0204 80.7978) (width 0.3) (layer "B.Cu") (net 24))
 (segment (start 85.1364 91.546) (end 86.6594 91.546) (width 0.5) (layer "B.Cu") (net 1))
 (segment (start 81.534 95.1484) (end 85.1364 91.546) (width 0.5) (layer "B.Cu") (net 1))
 (segment (start 88.9102 84.7852) (end 88.9102 87.9144) (width 0.5) (layer "B.Cu") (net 1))
 (segment (start 86.9848 84.7598) (end 87.0102 84.7852) (width 0.5) (layer "B.Cu") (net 1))
 (segment (start 80.8482 95.1484) (end 81.534 95.1484) (width 0.5) (layer "B.Cu") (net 1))
 (segment (start 87.0102 89.8144) (end 87.0102 91.1952) (width 0.5) (layer "B.Cu") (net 1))
 (segment (start 84.8396 84.7598) (end 84.8396 73.268) (width 0.3) (layer "B.Cu") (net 1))
 (segment (start 84.8396 73.268) (end 83.9108 72.3392) (width 0.3) (layer "B.Cu") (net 1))
 (segment (start 84.8396 84.7598) (end 86.9848 84.7598) (width 0.5) (layer "B.Cu") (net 1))
 (segment (start 87.0102 91.1952) (end 86.6594 91.546) (width 0.5) (layer "B.Cu") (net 1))
 (segment (start 88.9102 87.9144) (end 87.0102 89.8144) (width 0.5) (layer "B.Cu") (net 1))
 (segment (start 87.0102 84.7852) (end 87.0102 89.8144) (width 0.5) (layer "B.Cu") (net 1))
 (segment (start 87.0102 91.4238) (end 86.888 91.546) (width 0.5) (layer "B.Cu") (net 1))
 (segment (start 82.1436 70.5104) (end 79.8377 70.5104) (width 0.3) (layer "F.Cu") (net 3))
 (segment (start 79.8377 70.5104) (end 79.829 70.5191) (width 0.3) (layer "F.Cu") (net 3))
 (via (at 82.1436 70.5104) (size 0.8) (drill 0.3) (layers "F.Cu" "B.Cu") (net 3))
 (segment (start 83.9108 70.5142) (end 86.4108 70.5142) (width 0.3) (layer "B.Cu") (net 3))
 (segment (start 83.9108 70.5142) (end 82.1474 70.5142) (width 0.3) (layer "B.Cu") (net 3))
 (segment (start 82.1474 70.5142) (end 82.1436 70.5104) (width 0.3) (layer "B.Cu") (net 3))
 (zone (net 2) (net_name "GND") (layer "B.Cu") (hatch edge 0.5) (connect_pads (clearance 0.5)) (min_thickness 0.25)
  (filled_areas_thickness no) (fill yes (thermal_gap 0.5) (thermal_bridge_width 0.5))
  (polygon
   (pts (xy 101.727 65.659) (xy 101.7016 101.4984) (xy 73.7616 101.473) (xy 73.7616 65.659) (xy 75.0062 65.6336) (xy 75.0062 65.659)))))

